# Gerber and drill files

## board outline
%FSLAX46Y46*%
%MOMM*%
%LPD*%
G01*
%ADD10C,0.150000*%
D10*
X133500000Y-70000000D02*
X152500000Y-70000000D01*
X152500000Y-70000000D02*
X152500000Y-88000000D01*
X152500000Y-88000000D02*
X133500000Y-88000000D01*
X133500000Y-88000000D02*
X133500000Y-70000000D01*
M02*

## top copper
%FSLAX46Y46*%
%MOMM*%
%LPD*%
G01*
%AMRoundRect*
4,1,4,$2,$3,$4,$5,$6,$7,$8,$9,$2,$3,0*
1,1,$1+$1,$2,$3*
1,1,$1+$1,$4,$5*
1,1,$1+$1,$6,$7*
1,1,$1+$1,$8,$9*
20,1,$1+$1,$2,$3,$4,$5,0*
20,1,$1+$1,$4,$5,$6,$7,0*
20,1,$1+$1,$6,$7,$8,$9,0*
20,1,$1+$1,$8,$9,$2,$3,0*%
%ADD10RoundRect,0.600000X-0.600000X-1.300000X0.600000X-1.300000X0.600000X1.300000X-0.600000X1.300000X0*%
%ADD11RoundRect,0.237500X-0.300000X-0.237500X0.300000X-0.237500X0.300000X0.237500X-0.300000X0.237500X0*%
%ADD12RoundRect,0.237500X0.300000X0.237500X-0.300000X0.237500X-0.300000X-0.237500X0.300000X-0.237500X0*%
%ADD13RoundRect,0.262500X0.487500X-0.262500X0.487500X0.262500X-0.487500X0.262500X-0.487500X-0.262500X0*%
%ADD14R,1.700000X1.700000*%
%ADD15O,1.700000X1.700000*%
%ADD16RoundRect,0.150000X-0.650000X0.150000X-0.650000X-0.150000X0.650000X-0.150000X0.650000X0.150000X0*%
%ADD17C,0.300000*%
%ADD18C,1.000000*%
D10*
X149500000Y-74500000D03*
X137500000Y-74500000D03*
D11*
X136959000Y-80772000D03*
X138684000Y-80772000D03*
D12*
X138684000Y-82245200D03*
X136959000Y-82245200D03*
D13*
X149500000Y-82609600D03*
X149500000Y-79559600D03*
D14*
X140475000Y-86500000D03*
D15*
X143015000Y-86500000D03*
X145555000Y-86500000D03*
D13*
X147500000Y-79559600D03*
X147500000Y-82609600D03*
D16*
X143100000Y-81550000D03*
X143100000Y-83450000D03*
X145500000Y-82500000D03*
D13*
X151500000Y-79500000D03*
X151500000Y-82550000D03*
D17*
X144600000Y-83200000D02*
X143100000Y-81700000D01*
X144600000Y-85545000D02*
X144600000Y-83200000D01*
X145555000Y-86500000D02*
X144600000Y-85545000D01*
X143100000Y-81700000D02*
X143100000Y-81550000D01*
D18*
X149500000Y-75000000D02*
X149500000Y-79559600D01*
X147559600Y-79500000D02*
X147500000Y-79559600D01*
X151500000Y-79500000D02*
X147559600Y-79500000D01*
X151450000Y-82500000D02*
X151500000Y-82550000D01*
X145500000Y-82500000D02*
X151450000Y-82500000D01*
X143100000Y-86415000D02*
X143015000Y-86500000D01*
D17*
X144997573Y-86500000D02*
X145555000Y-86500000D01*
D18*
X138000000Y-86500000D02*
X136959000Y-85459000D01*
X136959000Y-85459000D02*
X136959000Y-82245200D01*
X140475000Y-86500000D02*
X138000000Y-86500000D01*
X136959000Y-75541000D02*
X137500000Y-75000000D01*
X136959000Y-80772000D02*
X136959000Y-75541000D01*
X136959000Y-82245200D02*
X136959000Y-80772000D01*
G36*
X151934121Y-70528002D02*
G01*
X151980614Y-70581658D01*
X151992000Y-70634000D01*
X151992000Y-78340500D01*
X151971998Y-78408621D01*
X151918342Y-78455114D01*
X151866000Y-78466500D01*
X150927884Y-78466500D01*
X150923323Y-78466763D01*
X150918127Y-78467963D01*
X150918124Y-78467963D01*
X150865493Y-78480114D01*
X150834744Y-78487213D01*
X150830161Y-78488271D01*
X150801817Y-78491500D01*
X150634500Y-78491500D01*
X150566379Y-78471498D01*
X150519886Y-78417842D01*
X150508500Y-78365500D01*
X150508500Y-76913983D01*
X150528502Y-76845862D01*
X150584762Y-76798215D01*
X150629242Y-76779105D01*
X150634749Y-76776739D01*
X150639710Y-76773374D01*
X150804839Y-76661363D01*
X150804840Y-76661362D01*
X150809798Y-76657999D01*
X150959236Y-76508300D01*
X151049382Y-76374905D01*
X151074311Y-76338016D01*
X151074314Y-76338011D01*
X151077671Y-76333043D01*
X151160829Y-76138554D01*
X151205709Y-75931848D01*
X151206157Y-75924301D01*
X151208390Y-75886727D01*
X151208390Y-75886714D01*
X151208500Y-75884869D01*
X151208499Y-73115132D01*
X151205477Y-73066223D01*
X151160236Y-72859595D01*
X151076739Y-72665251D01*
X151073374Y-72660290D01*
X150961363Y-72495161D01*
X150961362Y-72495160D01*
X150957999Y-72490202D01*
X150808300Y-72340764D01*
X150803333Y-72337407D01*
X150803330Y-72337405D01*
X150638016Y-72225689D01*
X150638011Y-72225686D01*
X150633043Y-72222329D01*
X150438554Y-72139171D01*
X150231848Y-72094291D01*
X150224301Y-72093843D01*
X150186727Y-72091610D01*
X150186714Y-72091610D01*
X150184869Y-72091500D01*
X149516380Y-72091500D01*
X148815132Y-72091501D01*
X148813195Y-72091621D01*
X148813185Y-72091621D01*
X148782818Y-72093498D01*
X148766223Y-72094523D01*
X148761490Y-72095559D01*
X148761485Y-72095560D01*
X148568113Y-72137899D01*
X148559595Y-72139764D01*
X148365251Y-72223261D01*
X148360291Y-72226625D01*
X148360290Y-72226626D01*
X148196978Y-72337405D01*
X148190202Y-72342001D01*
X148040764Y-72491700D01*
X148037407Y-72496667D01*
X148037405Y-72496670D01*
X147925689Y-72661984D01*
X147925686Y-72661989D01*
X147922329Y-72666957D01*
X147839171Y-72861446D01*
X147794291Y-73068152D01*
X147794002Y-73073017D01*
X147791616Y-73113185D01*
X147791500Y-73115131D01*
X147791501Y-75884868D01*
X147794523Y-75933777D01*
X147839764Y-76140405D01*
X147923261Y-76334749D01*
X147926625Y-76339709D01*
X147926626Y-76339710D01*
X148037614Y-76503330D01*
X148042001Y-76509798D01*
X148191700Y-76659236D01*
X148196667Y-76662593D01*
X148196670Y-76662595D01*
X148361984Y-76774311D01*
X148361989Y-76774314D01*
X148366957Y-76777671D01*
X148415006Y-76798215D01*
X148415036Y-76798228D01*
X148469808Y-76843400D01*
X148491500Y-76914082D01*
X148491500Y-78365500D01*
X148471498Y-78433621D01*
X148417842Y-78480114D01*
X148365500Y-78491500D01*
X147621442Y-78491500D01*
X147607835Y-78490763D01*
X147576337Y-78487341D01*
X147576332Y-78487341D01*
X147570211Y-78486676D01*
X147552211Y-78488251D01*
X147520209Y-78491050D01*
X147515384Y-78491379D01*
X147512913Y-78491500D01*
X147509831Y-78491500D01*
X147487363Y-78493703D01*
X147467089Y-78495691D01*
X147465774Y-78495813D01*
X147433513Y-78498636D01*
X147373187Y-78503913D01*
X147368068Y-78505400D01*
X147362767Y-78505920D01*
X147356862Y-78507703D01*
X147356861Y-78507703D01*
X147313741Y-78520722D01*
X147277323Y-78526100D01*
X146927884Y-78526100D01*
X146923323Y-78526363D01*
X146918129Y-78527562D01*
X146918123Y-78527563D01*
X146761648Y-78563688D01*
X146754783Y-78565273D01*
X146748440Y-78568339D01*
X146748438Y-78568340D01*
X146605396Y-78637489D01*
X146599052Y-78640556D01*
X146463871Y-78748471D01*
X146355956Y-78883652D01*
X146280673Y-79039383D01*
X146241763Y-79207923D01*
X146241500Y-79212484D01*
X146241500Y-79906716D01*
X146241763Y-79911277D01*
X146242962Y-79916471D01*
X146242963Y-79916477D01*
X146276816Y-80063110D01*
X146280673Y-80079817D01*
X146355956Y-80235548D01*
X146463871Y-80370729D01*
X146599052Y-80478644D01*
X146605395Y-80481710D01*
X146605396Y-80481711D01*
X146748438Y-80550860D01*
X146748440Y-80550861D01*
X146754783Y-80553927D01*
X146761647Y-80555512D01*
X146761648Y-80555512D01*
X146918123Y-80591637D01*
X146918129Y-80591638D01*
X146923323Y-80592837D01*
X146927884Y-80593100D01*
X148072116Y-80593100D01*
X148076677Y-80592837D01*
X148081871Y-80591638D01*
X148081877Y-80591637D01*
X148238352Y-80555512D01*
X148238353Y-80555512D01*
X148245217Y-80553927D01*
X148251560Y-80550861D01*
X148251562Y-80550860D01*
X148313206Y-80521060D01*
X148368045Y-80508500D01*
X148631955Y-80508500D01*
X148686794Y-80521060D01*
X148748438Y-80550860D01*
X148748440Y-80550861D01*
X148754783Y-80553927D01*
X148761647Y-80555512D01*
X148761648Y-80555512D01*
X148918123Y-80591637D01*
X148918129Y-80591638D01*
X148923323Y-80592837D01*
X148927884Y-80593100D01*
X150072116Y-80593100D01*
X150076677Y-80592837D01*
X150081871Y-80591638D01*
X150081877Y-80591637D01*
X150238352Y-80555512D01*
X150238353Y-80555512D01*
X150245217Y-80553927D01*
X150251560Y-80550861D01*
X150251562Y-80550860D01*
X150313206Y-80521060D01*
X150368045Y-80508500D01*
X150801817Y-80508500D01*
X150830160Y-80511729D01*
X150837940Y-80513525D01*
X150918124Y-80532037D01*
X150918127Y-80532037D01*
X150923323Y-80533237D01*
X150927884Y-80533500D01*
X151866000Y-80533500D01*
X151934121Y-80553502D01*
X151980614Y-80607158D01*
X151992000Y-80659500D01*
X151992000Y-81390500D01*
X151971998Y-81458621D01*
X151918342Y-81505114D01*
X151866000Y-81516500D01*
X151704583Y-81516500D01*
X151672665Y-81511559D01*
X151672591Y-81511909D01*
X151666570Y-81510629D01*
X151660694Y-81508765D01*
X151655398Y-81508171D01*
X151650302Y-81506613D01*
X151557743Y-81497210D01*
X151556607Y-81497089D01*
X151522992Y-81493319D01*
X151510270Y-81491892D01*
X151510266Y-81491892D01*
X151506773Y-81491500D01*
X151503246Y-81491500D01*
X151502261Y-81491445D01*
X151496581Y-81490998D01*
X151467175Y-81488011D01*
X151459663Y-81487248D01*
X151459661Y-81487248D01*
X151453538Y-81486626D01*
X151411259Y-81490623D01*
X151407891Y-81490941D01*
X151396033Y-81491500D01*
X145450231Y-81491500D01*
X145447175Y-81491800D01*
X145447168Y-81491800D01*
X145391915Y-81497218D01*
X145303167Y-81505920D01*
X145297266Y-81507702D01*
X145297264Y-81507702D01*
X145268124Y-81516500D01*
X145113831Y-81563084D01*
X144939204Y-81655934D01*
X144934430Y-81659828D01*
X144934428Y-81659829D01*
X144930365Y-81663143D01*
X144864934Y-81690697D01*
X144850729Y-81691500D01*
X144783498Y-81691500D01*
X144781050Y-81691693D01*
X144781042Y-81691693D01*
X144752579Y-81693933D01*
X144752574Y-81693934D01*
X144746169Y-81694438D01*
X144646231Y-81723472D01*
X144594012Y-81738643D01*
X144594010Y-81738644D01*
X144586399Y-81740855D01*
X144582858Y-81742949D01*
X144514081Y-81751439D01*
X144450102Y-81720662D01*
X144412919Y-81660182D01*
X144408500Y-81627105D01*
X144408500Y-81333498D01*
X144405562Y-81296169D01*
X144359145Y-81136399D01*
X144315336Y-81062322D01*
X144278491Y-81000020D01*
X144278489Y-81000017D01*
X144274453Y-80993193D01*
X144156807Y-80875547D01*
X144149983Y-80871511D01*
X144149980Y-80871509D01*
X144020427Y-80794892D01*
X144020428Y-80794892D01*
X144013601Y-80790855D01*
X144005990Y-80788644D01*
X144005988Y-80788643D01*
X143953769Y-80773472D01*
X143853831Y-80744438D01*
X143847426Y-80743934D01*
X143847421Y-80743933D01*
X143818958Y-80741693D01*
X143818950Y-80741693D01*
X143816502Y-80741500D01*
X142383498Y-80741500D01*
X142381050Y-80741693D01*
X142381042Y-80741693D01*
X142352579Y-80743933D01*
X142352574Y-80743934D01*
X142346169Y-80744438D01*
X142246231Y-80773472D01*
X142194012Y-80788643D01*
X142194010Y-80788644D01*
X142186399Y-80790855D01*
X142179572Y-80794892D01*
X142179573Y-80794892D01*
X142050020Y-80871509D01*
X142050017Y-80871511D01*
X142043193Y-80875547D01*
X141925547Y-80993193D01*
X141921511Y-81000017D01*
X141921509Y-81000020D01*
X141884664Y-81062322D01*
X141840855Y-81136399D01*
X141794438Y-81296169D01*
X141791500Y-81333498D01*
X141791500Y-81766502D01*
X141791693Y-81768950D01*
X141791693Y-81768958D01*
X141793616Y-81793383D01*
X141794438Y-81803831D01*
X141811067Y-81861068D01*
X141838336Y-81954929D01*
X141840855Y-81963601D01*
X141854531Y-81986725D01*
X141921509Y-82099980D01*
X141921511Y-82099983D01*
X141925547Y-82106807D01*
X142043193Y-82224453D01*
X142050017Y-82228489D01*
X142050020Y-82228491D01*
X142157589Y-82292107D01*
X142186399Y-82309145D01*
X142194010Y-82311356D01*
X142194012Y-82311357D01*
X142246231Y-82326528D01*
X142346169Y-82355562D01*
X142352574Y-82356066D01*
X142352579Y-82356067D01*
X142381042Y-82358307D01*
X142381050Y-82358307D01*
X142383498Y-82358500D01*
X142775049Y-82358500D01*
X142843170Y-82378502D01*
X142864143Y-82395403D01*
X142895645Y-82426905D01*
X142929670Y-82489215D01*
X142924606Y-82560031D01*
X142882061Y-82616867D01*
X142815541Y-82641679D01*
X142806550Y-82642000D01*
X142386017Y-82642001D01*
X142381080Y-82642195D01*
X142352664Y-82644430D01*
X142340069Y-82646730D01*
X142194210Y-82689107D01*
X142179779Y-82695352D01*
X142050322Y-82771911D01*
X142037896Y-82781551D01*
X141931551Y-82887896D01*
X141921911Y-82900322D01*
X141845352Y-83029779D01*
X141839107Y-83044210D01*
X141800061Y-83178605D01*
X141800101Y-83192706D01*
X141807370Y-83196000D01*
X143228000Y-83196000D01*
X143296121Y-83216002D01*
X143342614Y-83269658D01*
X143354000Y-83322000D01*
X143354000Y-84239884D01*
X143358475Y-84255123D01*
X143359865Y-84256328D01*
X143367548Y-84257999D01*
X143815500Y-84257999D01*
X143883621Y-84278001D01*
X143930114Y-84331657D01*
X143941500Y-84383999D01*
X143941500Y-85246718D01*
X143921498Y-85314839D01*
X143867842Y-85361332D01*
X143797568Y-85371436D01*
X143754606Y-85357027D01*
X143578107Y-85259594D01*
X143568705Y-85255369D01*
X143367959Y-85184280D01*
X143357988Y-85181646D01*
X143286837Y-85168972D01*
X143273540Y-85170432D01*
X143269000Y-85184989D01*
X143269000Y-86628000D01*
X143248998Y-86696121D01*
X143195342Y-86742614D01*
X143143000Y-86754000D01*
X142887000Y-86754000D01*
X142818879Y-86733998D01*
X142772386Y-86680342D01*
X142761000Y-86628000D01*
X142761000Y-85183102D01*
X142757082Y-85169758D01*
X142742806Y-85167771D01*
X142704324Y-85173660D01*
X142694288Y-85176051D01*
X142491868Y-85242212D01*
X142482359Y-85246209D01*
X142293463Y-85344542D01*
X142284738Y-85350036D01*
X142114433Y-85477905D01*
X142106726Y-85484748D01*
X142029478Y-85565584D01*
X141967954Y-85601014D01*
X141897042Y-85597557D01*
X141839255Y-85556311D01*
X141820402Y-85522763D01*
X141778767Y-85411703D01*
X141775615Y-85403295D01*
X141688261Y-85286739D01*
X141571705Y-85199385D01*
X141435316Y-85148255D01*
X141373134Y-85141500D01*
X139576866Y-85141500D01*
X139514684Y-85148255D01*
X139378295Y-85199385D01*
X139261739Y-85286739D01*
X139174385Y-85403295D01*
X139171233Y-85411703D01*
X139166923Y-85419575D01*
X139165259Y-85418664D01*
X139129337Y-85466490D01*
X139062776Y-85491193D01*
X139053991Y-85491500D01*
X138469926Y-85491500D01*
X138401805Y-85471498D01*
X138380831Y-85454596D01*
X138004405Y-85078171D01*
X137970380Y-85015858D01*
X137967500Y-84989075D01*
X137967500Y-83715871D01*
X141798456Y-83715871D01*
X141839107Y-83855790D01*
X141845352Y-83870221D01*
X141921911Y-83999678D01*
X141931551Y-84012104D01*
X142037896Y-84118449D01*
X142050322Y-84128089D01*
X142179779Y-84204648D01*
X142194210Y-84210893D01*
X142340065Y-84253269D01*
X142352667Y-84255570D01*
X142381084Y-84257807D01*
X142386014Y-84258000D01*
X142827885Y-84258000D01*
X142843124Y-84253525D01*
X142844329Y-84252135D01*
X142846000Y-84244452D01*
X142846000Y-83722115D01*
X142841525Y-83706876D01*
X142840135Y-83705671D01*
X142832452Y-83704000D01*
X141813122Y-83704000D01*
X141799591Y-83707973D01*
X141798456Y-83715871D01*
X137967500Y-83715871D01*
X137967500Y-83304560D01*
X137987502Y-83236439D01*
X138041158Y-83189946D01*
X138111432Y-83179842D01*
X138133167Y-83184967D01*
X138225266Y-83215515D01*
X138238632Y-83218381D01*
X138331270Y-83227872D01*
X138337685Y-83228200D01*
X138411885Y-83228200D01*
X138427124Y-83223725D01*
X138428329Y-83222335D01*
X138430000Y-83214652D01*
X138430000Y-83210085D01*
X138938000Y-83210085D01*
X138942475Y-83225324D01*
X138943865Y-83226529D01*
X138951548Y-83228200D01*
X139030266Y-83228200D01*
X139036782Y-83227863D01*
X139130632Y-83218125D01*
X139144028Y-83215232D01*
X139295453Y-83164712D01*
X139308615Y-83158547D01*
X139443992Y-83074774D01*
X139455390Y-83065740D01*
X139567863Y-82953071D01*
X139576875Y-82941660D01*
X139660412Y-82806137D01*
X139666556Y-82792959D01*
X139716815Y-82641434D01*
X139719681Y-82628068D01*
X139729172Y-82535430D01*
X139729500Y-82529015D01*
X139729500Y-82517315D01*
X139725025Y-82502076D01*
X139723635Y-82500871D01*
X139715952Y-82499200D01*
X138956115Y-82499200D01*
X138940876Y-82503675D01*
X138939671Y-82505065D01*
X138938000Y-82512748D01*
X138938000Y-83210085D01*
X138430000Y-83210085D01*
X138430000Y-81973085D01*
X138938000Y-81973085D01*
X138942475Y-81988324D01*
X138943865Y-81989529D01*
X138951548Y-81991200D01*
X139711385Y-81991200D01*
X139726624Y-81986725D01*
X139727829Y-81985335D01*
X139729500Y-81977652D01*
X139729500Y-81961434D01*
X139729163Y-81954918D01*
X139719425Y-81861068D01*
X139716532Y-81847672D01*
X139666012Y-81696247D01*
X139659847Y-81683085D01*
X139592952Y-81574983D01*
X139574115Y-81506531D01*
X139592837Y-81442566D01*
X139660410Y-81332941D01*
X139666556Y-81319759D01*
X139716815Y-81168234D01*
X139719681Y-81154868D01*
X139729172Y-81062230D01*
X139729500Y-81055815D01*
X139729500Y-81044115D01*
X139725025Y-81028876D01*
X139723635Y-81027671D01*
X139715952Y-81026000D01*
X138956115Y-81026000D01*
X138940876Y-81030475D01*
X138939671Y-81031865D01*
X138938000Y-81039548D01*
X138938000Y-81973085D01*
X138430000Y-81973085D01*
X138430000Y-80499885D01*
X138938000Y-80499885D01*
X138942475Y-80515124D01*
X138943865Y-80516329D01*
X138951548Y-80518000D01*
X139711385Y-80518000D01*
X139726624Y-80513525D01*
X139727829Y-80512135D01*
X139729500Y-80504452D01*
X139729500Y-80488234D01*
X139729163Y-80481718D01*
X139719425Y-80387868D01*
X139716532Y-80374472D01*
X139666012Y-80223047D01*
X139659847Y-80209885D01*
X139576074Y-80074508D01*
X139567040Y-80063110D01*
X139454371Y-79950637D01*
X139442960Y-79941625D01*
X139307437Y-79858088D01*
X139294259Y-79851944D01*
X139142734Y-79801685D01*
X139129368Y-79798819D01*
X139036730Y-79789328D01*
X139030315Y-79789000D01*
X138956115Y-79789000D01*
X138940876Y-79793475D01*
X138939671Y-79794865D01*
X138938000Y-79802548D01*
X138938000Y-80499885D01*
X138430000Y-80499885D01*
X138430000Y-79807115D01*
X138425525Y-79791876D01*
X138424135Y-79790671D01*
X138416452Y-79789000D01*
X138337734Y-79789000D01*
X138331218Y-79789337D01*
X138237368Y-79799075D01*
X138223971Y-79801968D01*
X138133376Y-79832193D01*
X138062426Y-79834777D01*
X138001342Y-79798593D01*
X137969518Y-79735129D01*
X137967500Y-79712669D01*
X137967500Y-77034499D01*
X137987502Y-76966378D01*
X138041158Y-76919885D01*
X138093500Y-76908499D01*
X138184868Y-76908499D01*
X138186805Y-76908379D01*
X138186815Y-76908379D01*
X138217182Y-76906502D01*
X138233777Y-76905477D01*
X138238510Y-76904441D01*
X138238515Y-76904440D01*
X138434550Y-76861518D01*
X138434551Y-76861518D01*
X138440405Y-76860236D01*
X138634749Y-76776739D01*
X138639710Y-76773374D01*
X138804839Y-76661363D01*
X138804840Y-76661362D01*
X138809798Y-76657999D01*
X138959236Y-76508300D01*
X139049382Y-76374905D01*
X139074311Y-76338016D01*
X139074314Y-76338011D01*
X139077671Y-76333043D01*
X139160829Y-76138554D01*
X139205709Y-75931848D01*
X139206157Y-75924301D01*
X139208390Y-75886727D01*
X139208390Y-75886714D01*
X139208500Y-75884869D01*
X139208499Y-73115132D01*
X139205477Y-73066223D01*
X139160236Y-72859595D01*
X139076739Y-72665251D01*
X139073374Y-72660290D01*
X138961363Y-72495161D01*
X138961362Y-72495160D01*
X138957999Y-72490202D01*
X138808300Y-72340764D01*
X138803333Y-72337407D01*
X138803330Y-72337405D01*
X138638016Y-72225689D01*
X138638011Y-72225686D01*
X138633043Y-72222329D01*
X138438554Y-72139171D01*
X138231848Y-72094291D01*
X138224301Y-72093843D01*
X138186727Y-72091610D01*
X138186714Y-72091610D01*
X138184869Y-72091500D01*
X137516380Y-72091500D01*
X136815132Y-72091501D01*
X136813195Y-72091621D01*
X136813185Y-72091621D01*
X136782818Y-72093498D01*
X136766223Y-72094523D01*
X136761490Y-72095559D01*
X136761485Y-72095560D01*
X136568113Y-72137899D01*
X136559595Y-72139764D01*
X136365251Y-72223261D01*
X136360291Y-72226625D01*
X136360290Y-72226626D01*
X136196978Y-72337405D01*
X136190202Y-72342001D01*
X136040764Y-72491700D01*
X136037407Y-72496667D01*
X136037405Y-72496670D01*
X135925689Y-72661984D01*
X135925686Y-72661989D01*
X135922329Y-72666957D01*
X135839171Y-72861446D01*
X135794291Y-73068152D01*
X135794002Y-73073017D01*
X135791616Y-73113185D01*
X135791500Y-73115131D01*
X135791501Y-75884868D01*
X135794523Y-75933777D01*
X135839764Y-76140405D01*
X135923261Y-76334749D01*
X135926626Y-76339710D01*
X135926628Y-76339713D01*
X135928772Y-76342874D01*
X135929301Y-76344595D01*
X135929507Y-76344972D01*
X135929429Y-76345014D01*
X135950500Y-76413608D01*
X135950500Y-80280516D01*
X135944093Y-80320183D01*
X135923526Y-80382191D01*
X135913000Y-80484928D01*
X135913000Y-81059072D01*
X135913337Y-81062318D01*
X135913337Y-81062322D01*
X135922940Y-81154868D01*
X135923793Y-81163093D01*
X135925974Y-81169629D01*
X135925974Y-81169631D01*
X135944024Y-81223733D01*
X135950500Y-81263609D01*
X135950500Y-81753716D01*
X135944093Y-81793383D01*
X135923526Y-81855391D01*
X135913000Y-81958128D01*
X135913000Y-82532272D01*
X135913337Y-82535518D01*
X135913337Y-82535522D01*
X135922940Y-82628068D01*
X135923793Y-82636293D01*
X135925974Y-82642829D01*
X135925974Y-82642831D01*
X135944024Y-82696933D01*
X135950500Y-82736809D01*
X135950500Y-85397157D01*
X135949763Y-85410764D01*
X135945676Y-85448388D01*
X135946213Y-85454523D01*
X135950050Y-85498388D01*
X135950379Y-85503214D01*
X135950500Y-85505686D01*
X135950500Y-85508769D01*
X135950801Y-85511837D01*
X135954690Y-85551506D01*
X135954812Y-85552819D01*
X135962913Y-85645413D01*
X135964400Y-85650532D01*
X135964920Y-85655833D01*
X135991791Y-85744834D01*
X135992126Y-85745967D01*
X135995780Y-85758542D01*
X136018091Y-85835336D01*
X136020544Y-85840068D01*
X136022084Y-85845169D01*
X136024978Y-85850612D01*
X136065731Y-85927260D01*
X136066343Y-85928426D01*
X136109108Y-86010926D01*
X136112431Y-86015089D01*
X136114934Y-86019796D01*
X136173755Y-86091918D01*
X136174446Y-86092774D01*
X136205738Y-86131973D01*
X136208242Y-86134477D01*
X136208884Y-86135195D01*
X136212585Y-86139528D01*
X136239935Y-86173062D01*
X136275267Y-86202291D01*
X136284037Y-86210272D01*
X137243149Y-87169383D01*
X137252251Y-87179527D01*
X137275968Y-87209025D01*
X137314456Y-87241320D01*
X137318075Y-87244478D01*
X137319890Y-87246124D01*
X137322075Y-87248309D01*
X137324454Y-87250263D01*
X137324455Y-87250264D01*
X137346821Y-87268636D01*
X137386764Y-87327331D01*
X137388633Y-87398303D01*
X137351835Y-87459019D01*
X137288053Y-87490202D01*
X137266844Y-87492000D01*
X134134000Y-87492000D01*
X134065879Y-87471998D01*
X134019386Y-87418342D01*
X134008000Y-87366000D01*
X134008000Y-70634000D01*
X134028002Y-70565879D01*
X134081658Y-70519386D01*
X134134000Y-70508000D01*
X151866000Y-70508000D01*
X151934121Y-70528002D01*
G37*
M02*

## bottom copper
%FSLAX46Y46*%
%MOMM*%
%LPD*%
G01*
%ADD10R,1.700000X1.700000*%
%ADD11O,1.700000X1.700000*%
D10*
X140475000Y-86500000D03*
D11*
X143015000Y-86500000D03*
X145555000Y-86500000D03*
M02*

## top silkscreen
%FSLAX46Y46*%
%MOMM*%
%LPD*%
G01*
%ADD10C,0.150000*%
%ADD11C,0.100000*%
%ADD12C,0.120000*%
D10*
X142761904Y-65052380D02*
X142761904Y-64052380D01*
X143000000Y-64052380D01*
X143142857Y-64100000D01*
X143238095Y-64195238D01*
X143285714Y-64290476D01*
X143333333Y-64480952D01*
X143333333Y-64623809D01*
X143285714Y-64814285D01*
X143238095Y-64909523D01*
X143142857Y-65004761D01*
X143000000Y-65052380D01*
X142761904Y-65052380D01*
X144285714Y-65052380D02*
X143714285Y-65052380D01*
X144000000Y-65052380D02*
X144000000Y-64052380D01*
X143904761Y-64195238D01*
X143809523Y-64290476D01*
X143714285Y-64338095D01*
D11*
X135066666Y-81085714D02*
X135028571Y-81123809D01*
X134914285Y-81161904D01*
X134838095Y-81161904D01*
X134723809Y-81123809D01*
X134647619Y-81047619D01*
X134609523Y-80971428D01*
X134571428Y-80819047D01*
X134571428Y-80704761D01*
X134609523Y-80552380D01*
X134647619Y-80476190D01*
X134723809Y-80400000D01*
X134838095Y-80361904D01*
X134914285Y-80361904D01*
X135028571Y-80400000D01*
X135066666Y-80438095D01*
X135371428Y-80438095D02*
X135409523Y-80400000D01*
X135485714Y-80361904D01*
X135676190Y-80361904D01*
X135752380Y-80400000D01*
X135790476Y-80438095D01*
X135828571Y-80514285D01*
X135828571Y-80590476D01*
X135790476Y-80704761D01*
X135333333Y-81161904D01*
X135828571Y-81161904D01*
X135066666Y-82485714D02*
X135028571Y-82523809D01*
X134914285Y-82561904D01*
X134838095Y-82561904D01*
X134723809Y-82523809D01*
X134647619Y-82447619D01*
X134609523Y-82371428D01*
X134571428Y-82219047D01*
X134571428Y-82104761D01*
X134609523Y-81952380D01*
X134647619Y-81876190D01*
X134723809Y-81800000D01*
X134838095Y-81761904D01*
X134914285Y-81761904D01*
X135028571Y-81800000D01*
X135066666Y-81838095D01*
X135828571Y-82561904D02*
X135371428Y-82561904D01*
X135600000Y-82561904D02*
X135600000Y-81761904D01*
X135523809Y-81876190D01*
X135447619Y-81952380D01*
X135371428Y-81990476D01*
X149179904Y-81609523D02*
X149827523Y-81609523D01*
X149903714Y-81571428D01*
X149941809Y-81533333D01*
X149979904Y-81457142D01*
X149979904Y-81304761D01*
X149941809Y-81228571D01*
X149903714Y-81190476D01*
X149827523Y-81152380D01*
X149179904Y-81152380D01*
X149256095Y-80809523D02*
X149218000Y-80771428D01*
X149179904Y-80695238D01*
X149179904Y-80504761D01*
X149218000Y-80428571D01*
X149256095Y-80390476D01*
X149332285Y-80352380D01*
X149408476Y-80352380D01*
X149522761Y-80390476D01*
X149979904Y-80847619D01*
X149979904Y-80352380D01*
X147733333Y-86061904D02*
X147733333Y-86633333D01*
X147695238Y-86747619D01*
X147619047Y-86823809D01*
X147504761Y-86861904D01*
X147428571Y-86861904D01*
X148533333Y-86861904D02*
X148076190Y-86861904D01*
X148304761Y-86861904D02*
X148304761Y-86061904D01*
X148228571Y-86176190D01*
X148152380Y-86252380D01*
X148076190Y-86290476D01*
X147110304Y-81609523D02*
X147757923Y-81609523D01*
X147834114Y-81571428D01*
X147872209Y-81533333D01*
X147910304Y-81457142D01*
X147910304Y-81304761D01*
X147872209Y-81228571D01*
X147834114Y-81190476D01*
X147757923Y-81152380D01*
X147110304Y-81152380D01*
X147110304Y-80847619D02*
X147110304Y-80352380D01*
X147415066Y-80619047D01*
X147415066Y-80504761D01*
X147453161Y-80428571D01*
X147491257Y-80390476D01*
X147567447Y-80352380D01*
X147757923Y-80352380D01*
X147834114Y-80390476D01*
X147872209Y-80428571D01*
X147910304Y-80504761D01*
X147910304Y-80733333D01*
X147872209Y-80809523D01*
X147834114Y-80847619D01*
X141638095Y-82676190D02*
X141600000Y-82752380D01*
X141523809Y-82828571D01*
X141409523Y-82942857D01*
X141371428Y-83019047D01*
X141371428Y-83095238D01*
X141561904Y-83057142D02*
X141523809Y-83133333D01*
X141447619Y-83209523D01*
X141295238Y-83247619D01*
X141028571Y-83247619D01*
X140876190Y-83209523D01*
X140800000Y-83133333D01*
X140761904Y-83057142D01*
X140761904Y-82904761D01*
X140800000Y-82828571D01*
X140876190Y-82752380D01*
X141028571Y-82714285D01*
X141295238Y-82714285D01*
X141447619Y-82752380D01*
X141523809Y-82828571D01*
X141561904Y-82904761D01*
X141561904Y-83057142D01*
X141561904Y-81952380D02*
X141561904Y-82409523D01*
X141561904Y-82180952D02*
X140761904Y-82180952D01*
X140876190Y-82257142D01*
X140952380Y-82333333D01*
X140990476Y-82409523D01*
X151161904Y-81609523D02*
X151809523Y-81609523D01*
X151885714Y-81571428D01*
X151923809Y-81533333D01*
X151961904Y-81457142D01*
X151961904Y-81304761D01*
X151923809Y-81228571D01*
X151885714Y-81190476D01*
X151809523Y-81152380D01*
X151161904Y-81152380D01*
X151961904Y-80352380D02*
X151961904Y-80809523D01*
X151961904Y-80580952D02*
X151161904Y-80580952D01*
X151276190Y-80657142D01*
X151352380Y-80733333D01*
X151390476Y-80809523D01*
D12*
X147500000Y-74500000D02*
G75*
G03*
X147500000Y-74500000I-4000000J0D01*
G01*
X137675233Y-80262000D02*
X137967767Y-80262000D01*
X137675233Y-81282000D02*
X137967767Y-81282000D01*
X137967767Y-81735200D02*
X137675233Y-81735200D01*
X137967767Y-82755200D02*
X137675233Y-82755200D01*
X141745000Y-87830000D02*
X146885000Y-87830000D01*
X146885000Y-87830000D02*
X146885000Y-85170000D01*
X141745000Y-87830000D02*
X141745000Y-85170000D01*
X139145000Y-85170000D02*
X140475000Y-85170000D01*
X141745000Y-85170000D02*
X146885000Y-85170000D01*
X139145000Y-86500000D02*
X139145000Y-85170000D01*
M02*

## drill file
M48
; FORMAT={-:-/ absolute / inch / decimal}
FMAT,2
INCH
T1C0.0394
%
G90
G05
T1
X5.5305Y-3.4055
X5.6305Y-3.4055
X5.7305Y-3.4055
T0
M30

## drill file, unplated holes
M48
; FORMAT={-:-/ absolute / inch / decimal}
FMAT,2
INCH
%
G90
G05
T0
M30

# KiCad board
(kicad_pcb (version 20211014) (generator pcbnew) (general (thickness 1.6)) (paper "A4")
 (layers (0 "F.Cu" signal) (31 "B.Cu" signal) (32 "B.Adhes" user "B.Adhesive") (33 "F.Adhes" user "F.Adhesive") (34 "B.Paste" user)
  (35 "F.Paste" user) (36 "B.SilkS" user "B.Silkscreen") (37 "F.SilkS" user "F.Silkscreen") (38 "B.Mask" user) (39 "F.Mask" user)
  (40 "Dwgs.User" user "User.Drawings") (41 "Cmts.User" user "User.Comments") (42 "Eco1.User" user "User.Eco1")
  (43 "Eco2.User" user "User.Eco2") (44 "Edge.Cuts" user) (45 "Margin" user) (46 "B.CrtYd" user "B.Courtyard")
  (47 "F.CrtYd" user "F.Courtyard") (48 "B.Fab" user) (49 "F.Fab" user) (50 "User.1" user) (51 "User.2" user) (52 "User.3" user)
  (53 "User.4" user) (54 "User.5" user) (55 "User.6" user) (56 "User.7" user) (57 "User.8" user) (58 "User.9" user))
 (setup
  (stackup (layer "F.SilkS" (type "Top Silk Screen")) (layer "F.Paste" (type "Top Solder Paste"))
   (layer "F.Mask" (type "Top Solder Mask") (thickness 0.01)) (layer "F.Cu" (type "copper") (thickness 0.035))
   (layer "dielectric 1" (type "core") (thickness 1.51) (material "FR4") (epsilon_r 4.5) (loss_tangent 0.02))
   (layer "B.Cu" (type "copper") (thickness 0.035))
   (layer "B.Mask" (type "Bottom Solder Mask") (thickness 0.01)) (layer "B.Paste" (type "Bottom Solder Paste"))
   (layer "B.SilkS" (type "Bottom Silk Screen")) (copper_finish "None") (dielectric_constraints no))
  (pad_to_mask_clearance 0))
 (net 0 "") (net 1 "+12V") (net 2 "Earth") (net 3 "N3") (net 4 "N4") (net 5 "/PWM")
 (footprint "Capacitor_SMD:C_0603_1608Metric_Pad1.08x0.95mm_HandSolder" (layer "F.Cu") (at 137.8215 80.772)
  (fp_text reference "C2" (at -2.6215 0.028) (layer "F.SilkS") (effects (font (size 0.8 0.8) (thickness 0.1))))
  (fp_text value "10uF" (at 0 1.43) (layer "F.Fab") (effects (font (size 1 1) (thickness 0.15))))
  (fp_line (start -0.146267 -0.51) (end 0.146267 -0.51) (layer "F.SilkS") (width 0.12))
  (fp_line (start -0.146267 0.51) (end 0.146267 0.51) (layer "F.SilkS") (width 0.12))
  (pad "1" smd roundrect locked (at -0.8625 0) (size 1.075 0.95) (layers "F.Cu" "F.Paste" "F.Mask") (roundrect_rratio 0.25) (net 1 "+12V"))
  (pad "2" smd roundrect locked (at 0.8625 0) (size 1.075 0.95) (layers "F.Cu" "F.Paste" "F.Mask") (roundrect_rratio 0.25) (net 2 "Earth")))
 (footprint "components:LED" (layer "F.Cu") (at 143.5 74.5)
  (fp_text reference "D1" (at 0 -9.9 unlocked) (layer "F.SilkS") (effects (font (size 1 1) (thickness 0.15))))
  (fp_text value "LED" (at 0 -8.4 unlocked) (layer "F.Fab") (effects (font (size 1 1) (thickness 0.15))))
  (fp_circle (center 0 0) (end 4 0) (layer "F.SilkS") (width 0.12) (fill none))
  (pad "1" smd roundrect (at 6 0) (size 2.4 3.8) (layers "F.Cu" "F.Paste" "F.Mask" "Dwgs.User") (roundrect_rratio 0.25) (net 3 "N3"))
  (pad "2" smd roundrect (at -6 0) (size 2.4 3.8) (layers "F.Cu" "F.Paste" "F.Mask") (roundrect_rratio 0.25) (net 1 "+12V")))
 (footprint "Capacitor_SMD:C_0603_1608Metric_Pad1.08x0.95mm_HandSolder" (layer "F.Cu") (at 137.8215 82.2452 180)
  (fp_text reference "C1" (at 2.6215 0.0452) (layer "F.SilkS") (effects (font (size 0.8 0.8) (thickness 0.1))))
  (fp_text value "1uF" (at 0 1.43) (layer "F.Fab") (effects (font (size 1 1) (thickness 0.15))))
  (fp_line (start -0.146267 0.51) (end 0.146267 0.51) (layer "F.SilkS") (width 0.12))
  (fp_line (start -0.146267 -0.51) (end 0.146267 -0.51) (layer "F.SilkS") (width 0.12))
  (pad "1" smd roundrect locked (at -0.8625 0 180) (size 1.075 0.95) (layers "F.Cu" "F.Paste" "F.Mask") (roundrect_rratio 0.25)
   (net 2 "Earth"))
  (pad "2" smd roundrect locked (at 0.8625 0 180) (size 1.075 0.95) (layers "F.Cu" "F.Paste" "F.Mask") (roundrect_rratio 0.25)
   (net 1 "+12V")))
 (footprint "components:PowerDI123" (layer "F.Cu") (at 149.5 81.0846 90)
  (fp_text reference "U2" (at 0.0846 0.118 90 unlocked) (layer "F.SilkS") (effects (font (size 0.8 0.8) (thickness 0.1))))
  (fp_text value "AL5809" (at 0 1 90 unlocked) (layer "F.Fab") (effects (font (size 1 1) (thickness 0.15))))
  (pad "1" smd roundrect (at 1.525 0 90) (size 1.05 1.5) (layers "F.Cu" "F.Paste" "F.Mask") (roundrect_rratio 0.25) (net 3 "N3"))
  (pad "2" smd roundrect (at -1.525 0 90) (size 1.05 1.5) (layers "F.Cu" "F.Paste" "F.Mask") (roundrect_rratio 0.25) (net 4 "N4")))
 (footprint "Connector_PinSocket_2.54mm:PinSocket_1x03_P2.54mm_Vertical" (layer "F.Cu") (at 140.475 86.5 90)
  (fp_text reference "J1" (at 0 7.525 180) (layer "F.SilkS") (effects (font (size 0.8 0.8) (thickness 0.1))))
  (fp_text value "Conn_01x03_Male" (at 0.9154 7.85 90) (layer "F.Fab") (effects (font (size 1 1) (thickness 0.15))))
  (fp_line (start -1.33 1.27) (end -1.33 6.41) (layer "F.SilkS") (width 0.12))
  (fp_line (start -1.33 6.41) (end 1.33 6.41) (layer "F.SilkS") (width 0.12))
  (fp_line (start -1.33 1.27) (end 1.33 1.27) (layer "F.SilkS") (width 0.12))
  (fp_line (start 1.33 -1.33) (end 1.33 0) (layer "F.SilkS") (width 0.12))
  (fp_line (start 1.33 1.27) (end 1.33 6.41) (layer "F.SilkS") (width 0.12))
  (fp_line (start 0 -1.33) (end 1.33 -1.33) (layer "F.SilkS") (width 0.12))
  (pad "1" thru_hole rect locked (at 0 0 90) (size 1.7 1.7) (drill 1) (layers *.Cu *.Mask) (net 1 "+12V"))
  (pad "2" thru_hole oval locked (at 0 2.54 90) (size 1.7 1.7) (drill 1) (layers *.Cu *.Mask) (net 2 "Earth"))
  (pad "3" thru_hole oval locked (at 0 5.08 90) (size 1.7 1.7) (drill 1) (layers *.Cu *.Mask) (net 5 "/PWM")))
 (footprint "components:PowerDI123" (layer "F.Cu") (at 147.5 81.0846 90)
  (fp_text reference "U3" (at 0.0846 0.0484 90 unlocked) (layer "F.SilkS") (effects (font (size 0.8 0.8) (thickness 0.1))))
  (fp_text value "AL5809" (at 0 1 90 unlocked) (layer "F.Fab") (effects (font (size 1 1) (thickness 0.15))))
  (pad "1" smd roundrect (at 1.525 0 90) (size 1.05 1.5) (layers "F.Cu" "F.Paste" "F.Mask") (roundrect_rratio 0.25) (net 3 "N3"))
  (pad "2" smd roundrect (at -1.525 0 90) (size 1.05 1.5) (layers "F.Cu" "F.Paste" "F.Mask") (roundrect_rratio 0.25) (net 4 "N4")))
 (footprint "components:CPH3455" (layer "F.Cu") (at 143.1 82.5 -90)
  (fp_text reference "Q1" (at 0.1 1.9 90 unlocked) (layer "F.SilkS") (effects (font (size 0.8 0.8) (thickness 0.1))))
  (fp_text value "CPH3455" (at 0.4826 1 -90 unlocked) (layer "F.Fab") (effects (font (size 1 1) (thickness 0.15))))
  (pad "1" smd roundrect (at -0.95 0 270) (size 0.6 1.6) (layers "F.Cu" "F.Paste" "F.Mask") (roundrect_rratio 0.25) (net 5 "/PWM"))
  (pad "2" smd roundrect (at 0.95 0 270) (size 0.6 1.6) (layers "F.Cu" "F.Paste" "F.Mask") (roundrect_rratio 0.25) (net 2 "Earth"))
  (pad "3" smd roundrect (at 0 -2.4 270) (size 0.6 1.6) (layers "F.Cu" "F.Paste" "F.Mask") (roundrect_rratio 0.25) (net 4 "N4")))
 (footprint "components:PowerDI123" (layer "F.Cu") (at 151.5 81.025 90)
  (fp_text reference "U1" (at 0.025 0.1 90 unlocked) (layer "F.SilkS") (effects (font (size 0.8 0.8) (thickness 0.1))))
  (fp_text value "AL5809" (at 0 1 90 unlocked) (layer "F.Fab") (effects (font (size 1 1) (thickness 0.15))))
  (pad "1" smd roundrect (at 1.525 0 90) (size 1.05 1.5) (layers "F.Cu" "F.Paste" "F.Mask") (roundrect_rratio 0.25) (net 3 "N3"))
  (pad "2" smd roundrect (at -1.525 0 90) (size 1.05 1.5) (layers "F.Cu" "F.Paste" "F.Mask") (roundrect_rratio 0.25) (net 4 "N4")))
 (gr_rect (start 133.5 70) (end 152.5 88) (layer "Edge.Cuts") (width 0.15) (fill none))
 (segment (start 143.1 86.415) (end 143.015 86.5) (width 1) (layer "F.Cu") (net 2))
 (segment (start 136.959 85.459) (end 136.959 82.2452) (width 1) (layer "F.Cu") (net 1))
 (segment (start 138 86.5) (end 136.959 85.459) (width 1) (layer "F.Cu") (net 1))
 (segment (start 136.959 82.2452) (end 136.959 80.772) (width 1) (layer "F.Cu") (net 1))
 (segment (start 136.959 80.772) (end 136.959 75.541) (width 1) (layer "F.Cu") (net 1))
 (segment (start 136.959 75.541) (end 137.5 75) (width 1) (layer "F.Cu") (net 1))
 (segment (start 140.475 86.5) (end 138 86.5) (width 1) (layer "F.Cu") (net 1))
 (segment (start 151.5 79.5) (end 147.5596 79.5) (width 1) (layer "F.Cu") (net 3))
 (segment (start 147.5596 79.5) (end 147.5 79.5596) (width 1) (layer "F.Cu") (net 3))
 (segment (start 149.5 75) (end 149.5 79.5596) (width 1) (layer "F.Cu") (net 3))
 (segment (start 143.1 81.7) (end 143.1 81.55) (width 0.3) (layer "F.Cu") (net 5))
 (segment (start 144.6 85.545) (end 144.6 83.2) (width 0.3) (layer "F.Cu") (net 5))
 (segment (start 145.555 86.5) (end 144.6 85.545) (width 0.3) (layer "F.Cu") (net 5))
 (segment (start 144.997573 86.5) (end 145.555 86.5) (width 0.3) (layer "F.Cu") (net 5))
 (segment (start 144.6 83.2) (end 143.1 81.7) (width 0.3) (layer "F.Cu") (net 5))
 (segment (start 145.5 82.5) (end 151.45 82.5) (width 1) (layer "F.Cu") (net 4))
 (segment (start 151.45 82.5) (end 151.5 82.55) (width 1) (layer "F.Cu") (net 4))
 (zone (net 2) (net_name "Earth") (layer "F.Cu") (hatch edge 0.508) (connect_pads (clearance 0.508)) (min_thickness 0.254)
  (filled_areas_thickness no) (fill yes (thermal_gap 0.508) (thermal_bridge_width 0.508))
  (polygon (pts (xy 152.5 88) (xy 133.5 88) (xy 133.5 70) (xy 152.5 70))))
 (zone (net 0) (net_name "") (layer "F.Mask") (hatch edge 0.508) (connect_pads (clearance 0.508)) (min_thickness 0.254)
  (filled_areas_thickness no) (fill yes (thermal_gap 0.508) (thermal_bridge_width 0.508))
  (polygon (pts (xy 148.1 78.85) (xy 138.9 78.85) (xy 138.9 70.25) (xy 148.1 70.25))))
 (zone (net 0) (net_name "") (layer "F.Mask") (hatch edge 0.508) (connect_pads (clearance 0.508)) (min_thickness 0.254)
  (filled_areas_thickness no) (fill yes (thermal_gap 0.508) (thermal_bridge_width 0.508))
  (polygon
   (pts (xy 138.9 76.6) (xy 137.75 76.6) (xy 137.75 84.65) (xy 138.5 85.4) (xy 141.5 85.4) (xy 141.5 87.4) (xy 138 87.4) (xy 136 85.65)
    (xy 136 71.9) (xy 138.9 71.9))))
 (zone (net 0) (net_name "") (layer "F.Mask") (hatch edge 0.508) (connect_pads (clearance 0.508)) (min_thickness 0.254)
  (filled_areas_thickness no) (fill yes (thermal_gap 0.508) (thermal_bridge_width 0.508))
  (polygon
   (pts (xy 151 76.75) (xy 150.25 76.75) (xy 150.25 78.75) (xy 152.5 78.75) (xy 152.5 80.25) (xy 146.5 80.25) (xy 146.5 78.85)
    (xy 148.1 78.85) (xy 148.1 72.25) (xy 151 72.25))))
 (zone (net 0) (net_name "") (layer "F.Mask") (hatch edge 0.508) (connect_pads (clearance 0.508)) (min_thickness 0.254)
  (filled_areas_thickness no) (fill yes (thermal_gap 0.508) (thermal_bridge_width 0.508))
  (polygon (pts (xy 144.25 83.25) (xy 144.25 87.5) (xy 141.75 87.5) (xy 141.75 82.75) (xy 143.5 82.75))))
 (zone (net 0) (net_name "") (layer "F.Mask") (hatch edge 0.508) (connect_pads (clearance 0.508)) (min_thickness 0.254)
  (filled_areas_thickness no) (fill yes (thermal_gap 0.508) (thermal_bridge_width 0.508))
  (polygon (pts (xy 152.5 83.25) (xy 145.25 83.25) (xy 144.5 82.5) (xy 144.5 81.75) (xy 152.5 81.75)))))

